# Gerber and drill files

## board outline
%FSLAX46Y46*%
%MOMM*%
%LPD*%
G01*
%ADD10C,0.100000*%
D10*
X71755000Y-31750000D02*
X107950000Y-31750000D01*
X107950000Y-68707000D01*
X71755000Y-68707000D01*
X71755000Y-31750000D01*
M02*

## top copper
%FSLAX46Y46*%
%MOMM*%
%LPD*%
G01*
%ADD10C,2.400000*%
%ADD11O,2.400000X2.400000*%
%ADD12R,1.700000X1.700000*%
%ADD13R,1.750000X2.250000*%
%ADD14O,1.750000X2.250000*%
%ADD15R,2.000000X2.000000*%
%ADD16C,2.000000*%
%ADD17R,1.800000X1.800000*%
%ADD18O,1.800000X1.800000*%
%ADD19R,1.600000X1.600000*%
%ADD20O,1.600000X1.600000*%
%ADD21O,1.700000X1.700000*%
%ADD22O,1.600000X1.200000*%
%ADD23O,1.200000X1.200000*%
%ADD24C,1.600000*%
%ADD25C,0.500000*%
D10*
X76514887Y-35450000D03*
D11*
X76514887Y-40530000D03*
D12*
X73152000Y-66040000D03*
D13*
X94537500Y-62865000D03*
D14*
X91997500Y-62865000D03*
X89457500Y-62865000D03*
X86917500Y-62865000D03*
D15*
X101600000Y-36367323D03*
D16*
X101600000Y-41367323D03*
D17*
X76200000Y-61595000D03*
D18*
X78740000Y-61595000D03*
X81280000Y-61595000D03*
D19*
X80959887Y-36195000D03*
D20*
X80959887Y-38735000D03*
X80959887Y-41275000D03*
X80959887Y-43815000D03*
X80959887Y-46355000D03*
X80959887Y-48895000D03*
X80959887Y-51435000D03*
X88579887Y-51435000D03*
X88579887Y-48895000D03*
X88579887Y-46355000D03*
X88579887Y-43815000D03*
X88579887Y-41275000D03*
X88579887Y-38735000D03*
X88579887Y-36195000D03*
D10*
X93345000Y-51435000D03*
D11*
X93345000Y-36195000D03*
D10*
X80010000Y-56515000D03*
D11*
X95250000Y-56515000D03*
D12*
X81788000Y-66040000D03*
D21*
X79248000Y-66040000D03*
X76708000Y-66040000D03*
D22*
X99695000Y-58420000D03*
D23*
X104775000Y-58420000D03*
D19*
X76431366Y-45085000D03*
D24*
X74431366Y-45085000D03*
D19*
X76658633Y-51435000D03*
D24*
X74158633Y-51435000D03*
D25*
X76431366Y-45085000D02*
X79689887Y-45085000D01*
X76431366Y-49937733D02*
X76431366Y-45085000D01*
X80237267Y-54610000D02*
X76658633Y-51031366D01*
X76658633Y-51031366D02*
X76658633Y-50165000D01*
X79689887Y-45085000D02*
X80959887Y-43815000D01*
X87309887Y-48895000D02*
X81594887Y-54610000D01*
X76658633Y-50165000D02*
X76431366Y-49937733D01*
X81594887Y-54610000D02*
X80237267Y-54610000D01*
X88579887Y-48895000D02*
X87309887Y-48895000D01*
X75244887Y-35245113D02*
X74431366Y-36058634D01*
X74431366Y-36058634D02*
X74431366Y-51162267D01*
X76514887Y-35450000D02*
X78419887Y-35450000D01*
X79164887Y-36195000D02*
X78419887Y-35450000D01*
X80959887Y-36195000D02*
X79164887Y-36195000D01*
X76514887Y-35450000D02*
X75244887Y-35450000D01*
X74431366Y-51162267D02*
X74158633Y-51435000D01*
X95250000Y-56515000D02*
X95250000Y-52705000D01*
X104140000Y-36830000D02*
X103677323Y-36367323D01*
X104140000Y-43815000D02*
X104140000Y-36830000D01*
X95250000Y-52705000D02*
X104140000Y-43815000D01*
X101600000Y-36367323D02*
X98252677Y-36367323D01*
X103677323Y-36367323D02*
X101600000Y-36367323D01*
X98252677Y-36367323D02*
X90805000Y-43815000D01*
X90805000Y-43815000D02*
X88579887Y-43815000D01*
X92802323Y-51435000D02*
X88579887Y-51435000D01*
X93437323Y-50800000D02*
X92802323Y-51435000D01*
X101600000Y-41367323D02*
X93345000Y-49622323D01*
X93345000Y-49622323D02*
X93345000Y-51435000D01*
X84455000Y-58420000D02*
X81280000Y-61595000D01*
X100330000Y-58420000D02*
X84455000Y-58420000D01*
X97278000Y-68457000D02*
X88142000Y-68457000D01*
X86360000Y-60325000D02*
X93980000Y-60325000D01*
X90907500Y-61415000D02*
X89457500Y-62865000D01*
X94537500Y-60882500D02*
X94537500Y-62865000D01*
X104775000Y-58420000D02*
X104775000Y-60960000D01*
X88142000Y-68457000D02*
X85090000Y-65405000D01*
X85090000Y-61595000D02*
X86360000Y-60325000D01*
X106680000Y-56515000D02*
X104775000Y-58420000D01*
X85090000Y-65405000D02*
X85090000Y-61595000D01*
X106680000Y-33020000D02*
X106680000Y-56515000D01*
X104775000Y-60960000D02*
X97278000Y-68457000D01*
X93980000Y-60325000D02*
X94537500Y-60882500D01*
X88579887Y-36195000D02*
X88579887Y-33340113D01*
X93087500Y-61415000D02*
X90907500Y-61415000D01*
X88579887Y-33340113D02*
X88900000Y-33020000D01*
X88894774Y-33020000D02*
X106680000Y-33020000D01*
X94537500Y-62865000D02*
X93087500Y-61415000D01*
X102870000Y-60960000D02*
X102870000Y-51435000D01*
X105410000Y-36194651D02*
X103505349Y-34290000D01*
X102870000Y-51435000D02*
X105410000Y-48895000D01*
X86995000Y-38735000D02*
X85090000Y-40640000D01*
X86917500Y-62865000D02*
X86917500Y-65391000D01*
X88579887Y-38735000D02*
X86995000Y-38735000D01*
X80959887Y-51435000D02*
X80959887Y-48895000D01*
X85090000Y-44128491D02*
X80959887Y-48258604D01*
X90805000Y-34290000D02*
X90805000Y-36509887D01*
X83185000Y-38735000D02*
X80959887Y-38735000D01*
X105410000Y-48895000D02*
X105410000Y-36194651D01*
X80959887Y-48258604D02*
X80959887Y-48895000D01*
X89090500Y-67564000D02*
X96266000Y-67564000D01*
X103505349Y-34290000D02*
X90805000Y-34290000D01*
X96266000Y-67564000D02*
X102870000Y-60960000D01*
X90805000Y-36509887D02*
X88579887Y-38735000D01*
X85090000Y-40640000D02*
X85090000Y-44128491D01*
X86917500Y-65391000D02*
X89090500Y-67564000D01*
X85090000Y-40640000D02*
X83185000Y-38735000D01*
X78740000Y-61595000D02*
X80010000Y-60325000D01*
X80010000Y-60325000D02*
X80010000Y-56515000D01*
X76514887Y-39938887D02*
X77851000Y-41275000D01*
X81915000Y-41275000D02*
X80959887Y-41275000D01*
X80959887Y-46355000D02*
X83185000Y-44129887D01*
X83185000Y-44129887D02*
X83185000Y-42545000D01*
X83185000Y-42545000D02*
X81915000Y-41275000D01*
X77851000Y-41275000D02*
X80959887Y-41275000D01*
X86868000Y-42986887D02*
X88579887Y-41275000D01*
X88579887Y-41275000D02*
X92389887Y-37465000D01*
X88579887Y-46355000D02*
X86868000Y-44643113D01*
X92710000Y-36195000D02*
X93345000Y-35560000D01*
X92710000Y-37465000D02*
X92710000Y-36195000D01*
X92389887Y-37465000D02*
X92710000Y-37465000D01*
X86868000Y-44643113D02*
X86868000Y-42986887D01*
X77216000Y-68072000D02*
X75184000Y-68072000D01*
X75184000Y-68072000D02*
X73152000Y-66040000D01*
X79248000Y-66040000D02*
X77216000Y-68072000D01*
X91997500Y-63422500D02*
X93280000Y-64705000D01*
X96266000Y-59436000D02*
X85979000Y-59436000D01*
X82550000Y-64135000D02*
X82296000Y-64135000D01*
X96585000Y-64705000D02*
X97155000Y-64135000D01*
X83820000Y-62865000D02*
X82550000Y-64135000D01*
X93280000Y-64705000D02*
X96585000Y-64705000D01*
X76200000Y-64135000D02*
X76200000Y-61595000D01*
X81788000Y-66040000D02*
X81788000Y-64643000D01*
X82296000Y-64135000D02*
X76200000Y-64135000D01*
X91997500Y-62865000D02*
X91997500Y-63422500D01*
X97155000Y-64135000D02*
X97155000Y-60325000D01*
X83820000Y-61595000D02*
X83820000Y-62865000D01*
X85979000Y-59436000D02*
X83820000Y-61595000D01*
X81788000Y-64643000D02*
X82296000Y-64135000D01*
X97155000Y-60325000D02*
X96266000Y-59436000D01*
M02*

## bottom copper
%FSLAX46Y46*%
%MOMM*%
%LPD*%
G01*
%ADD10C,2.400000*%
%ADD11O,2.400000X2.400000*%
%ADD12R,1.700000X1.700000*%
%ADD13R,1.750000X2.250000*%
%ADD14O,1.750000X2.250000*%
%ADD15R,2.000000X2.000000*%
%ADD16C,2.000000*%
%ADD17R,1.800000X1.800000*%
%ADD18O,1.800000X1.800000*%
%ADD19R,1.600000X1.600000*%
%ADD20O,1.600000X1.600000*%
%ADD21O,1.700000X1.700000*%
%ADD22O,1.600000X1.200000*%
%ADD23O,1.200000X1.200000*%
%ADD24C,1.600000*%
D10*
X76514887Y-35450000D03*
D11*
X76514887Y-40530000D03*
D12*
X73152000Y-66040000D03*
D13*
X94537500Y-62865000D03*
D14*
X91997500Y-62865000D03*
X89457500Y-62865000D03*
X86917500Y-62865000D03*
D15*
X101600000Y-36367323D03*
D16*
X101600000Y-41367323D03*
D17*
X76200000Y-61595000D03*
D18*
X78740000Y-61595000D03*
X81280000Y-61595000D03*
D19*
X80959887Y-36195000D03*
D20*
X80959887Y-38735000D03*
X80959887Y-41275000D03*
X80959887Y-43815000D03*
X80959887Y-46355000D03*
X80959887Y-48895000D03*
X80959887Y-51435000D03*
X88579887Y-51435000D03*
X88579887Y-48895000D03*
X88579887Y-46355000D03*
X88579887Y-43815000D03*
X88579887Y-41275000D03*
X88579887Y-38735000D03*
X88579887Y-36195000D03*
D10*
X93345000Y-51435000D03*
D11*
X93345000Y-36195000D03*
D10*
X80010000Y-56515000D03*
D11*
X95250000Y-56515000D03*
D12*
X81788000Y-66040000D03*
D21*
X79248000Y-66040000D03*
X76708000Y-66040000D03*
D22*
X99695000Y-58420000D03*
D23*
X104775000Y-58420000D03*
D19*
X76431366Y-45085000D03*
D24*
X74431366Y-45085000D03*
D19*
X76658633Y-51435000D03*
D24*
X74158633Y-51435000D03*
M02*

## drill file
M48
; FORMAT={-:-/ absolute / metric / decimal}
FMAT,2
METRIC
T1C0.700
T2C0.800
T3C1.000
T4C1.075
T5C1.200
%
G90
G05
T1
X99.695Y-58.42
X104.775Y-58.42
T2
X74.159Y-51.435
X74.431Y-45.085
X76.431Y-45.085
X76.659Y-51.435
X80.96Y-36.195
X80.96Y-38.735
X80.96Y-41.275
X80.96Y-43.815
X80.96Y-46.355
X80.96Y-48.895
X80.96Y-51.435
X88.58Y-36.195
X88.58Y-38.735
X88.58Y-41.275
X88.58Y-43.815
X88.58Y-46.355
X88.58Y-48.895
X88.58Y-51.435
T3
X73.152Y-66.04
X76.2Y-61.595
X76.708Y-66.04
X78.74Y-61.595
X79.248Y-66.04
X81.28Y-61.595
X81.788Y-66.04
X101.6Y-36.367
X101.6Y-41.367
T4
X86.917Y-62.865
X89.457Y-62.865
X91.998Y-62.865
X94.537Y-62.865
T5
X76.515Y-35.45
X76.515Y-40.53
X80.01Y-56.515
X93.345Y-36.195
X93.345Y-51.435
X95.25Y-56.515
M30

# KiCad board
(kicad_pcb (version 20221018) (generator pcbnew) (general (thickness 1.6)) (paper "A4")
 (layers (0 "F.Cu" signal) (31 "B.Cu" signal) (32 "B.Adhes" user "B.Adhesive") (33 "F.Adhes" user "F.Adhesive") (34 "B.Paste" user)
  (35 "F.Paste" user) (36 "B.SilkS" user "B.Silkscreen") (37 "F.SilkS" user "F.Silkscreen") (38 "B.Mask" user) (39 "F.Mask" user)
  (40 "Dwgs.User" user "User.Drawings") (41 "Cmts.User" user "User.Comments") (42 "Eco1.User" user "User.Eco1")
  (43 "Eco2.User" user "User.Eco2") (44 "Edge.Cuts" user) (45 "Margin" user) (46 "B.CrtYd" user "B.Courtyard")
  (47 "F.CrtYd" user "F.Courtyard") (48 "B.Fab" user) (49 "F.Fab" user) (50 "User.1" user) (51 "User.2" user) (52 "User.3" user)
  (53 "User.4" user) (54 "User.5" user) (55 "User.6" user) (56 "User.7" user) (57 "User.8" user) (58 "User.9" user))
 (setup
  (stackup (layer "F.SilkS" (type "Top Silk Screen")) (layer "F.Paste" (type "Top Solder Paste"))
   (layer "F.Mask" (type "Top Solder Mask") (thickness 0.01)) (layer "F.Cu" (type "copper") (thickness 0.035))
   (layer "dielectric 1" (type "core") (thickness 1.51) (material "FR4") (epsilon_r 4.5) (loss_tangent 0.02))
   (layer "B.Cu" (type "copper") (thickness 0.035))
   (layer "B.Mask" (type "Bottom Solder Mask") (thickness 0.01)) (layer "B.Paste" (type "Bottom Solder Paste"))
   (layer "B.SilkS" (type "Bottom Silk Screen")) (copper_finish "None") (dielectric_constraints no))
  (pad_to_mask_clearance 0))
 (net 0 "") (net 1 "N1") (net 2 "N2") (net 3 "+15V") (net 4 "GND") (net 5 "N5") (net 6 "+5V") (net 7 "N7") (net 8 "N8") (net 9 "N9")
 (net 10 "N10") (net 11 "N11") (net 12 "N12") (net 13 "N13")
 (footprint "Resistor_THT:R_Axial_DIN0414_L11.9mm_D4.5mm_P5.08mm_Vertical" (layer "F.Cu") (at 76.514887 35.45 -90)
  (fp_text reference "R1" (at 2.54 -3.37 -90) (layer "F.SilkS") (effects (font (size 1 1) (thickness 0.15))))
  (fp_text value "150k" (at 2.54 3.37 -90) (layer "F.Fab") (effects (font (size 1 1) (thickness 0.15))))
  (pad "1" thru_hole circle (at 0 0 270) (size 2.4 2.4) (drill 1.2) (layers "*.Cu" "*.Mask") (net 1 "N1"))
  (pad "2" thru_hole oval (at 5.08 0 270) (size 2.4 2.4) (drill 1.2) (layers "*.Cu" "*.Mask") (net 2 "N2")))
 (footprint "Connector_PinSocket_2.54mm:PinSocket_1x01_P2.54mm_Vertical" (layer "F.Cu") (at 73.152 66.04)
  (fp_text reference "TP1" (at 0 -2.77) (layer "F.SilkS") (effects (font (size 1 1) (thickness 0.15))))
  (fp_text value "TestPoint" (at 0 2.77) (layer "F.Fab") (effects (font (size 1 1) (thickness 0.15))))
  (pad "1" thru_hole rect (at 0 0) (size 1.7 1.7) (drill 1) (layers "*.Cu" "*.Mask") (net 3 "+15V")))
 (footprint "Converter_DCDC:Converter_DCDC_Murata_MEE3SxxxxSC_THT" (layer "F.Cu") (at 94.5375 62.865 -90)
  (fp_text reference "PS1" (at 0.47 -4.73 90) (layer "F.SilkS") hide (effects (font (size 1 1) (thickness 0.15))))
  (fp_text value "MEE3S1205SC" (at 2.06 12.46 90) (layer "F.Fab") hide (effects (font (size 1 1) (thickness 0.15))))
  (pad "1" thru_hole rect (at 0 0 180) (size 1.75 2.25) (drill 1.075) (layers "*.Cu" "*.Mask") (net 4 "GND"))
  (pad "2" thru_hole oval (at 0 2.54 180) (size 1.75 2.25) (drill 1.075) (layers "*.Cu" "*.Mask") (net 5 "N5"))
  (pad "3" thru_hole oval (at 0 5.08 180) (size 1.75 2.25) (drill 1.075) (layers "*.Cu" "*.Mask") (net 4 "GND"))
  (pad "4" thru_hole oval (at 0 7.62 180) (size 1.75 2.25) (drill 1.075) (layers "*.Cu" "*.Mask") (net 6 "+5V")))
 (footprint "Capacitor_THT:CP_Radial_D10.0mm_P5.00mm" (layer "F.Cu") (at 101.6 36.367323 -90)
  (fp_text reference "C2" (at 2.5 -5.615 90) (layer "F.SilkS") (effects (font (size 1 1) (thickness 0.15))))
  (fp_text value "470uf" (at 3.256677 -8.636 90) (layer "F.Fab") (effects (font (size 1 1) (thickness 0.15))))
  (pad "1" thru_hole rect (at 0 0 270) (size 2 2) (drill 1) (layers "*.Cu" "*.Mask") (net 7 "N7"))
  (pad "2" thru_hole circle (at 5 0 270) (size 2 2) (drill 1) (layers "*.Cu" "*.Mask") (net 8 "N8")))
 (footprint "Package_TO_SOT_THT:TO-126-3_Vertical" (layer "F.Cu") (at 76.2 61.595)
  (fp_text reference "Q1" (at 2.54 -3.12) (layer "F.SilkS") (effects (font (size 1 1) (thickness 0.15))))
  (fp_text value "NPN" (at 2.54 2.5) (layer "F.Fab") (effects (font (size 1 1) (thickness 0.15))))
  (pad "1" thru_hole rect (at 0 0) (size 1.8 1.8) (drill 1) (layers "*.Cu" "*.Mask") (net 5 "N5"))
  (pad "2" thru_hole oval (at 2.54 0) (size 1.8 1.8) (drill 1) (layers "*.Cu" "*.Mask") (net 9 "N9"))
  (pad "3" thru_hole oval (at 5.08 0) (size 1.8 1.8) (drill 1) (layers "*.Cu" "*.Mask") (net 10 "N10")))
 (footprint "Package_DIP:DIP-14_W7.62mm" (layer "F.Cu") (at 80.959887 36.195)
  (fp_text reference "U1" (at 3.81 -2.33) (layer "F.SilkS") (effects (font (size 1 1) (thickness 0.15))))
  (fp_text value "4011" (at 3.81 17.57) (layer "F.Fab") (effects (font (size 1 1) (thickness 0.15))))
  (pad "1" thru_hole rect (at 0 0) (size 1.6 1.6) (drill 0.8) (layers "*.Cu" "*.Mask") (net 1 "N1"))
  (pad "2" thru_hole oval (at 0 2.54) (size 1.6 1.6) (drill 0.8) (layers "*.Cu" "*.Mask") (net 6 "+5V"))
  (pad "3" thru_hole oval (at 0 5.08) (size 1.6 1.6) (drill 0.8) (layers "*.Cu" "*.Mask") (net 2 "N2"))
  (pad "4" thru_hole oval (at 0 7.62) (size 1.6 1.6) (drill 0.8) (layers "*.Cu" "*.Mask") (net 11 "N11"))
  (pad "5" thru_hole oval (at 0 10.16) (size 1.6 1.6) (drill 0.8) (layers "*.Cu" "*.Mask") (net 2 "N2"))
  (pad "6" thru_hole oval (at 0 12.7) (size 1.6 1.6) (drill 0.8) (layers "*.Cu" "*.Mask") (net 6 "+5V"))
  (pad "7" thru_hole oval (at 0 15.24) (size 1.6 1.6) (drill 0.8) (layers "*.Cu" "*.Mask") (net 6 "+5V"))
  (pad "8" thru_hole oval (at 7.62 15.24) (size 1.6 1.6) (drill 0.8) (layers "*.Cu" "*.Mask") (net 8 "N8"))
  (pad "9" thru_hole oval (at 7.62 12.7) (size 1.6 1.6) (drill 0.8) (layers "*.Cu" "*.Mask") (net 11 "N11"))
  (pad "10" thru_hole oval (at 7.62 10.16) (size 1.6 1.6) (drill 0.8) (layers "*.Cu" "*.Mask") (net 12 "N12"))
  (pad "11" thru_hole oval (at 7.62 7.62) (size 1.6 1.6) (drill 0.8) (layers "*.Cu" "*.Mask") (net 7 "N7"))
  (pad "12" thru_hole oval (at 7.62 5.08) (size 1.6 1.6) (drill 0.8) (layers "*.Cu" "*.Mask") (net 12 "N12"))
  (pad "13" thru_hole oval (at 7.62 2.54) (size 1.6 1.6) (drill 0.8) (layers "*.Cu" "*.Mask") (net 6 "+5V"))
  (pad "14" thru_hole oval (at 7.62 0) (size 1.6 1.6) (drill 0.8) (layers "*.Cu" "*.Mask") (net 4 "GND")))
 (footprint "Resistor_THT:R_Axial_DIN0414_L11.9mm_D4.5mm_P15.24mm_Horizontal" (layer "F.Cu") (at 93.345 51.435 90)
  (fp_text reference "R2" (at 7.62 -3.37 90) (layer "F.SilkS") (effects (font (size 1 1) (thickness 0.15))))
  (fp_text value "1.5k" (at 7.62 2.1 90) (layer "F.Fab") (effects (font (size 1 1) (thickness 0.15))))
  (pad "1" thru_hole circle (at 0 0 90) (size 2.4 2.4) (drill 1.2) (layers "*.Cu" "*.Mask") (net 8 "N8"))
  (pad "2" thru_hole oval (at 15.24 0 90) (size 2.4 2.4) (drill 1.2) (layers "*.Cu" "*.Mask") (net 12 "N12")))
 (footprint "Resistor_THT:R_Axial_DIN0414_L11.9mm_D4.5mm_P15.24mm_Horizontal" (layer "F.Cu") (at 80.01 56.515)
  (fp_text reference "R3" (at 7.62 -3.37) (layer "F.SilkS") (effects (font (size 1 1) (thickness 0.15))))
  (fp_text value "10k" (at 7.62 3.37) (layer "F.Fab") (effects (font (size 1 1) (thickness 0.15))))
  (pad "1" thru_hole circle (at 0 0) (size 2.4 2.4) (drill 1.2) (layers "*.Cu" "*.Mask") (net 9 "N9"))
  (pad "2" thru_hole oval (at 15.24 0) (size 2.4 2.4) (drill 1.2) (layers "*.Cu" "*.Mask") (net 7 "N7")))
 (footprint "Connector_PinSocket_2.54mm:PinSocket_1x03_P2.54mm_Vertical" (layer "F.Cu") (at 81.788 66.04 -90)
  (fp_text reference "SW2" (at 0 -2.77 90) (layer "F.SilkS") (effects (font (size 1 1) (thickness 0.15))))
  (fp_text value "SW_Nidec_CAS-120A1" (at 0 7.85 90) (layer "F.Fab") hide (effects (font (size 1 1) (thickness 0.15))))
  (pad "1" thru_hole rect (at 0 0 270) (size 1.7 1.7) (drill 1) (layers "*.Cu" "*.Mask") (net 5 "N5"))
  (pad "2" thru_hole oval (at 0 2.54 270) (size 1.7 1.7) (drill 1) (layers "*.Cu" "*.Mask") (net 3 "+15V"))
  (pad "3" thru_hole oval (at 0 5.08 270) (size 1.7 1.7) (drill 1) (layers "*.Cu" "*.Mask") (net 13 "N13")))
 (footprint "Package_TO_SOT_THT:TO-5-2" (layer "F.Cu") (at 99.695 58.42)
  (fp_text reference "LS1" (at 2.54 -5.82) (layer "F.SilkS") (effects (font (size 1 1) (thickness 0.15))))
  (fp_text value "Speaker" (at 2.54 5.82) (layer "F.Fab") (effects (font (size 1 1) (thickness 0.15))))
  (pad "1" thru_hole oval (at 0 0) (size 1.6 1.2) (drill 0.7) (layers "*.Cu" "*.Mask") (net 10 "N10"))
  (pad "2" thru_hole oval (at 5.08 0) (size 1.2 1.2) (drill 0.7) (layers "*.Cu" "*.Mask") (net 4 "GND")))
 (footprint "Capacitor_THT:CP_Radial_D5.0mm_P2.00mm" (layer "F.Cu") (at 76.431366 45.085 180)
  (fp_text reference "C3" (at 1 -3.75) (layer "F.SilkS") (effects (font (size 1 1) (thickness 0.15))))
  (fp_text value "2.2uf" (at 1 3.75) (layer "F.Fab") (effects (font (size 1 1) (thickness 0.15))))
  (pad "1" thru_hole rect (at 0 0 180) (size 1.6 1.6) (drill 0.8) (layers "*.Cu" "*.Mask") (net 11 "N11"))
  (pad "2" thru_hole circle (at 2 0 180) (size 1.6 1.6) (drill 0.8) (layers "*.Cu" "*.Mask") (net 1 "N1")))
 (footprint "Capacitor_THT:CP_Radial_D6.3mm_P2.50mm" (layer "F.Cu") (at 76.658633 51.435 180)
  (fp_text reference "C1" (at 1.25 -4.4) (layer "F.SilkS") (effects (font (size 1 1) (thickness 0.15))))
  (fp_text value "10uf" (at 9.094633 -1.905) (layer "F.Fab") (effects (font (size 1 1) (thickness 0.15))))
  (pad "1" thru_hole rect (at 0 0 180) (size 1.6 1.6) (drill 0.8) (layers "*.Cu" "*.Mask") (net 11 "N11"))
  (pad "2" thru_hole circle (at 2.5 0 180) (size 1.6 1.6) (drill 0.8) (layers "*.Cu" "*.Mask") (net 1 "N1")))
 (gr_rect (start 71.755 31.75) (end 107.95 68.707) (stroke (width 0.1) (type default)) (fill none) (layer "Edge.Cuts"))
 (segment (start 76.431366 45.085) (end 79.689887 45.085) (width 0.5) (layer "F.Cu") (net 11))
 (segment (start 76.431366 49.937733) (end 76.431366 45.085) (width 0.5) (layer "F.Cu") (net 11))
 (segment (start 80.237267 54.61) (end 76.658633 51.031366) (width 0.5) (layer "F.Cu") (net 11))
 (segment (start 76.658633 51.031366) (end 76.658633 50.165) (width 0.5) (layer "F.Cu") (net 11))
 (segment (start 79.689887 45.085) (end 80.959887 43.815) (width 0.5) (layer "F.Cu") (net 11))
 (segment (start 87.309887 48.895) (end 81.594887 54.61) (width 0.5) (layer "F.Cu") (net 11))
 (segment (start 76.658633 50.165) (end 76.431366 49.937733) (width 0.5) (layer "F.Cu") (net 11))
 (segment (start 81.594887 54.61) (end 80.237267 54.61) (width 0.5) (layer "F.Cu") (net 11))
 (segment (start 88.579887 48.895) (end 87.309887 48.895) (width 0.5) (layer "F.Cu") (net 11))
 (segment (start 75.244887 35.245113) (end 74.431366 36.058634) (width 0.5) (layer "F.Cu") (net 1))
 (segment (start 74.431366 36.058634) (end 74.431366 51.162267) (width 0.5) (layer "F.Cu") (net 1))
 (segment (start 76.514887 35.45) (end 78.419887 35.45) (width 0.5) (layer "F.Cu") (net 1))
 (segment (start 79.164887 36.195) (end 78.419887 35.45) (width 0.5) (layer "F.Cu") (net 1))
 (segment (start 80.959887 36.195) (end 79.164887 36.195) (width 0.5) (layer "F.Cu") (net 1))
 (segment (start 76.514887 35.45) (end 75.244887 35.45) (width 0.5) (layer "F.Cu") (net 1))
 (segment (start 74.431366 51.162267) (end 74.158633 51.435) (width 0.5) (layer "F.Cu") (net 1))
 (segment (start 95.25 56.515) (end 95.25 52.705) (width 0.5) (layer "F.Cu") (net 7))
 (segment (start 104.14 36.83) (end 103.677323 36.367323) (width 0.5) (layer "F.Cu") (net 7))
 (segment (start 104.14 43.815) (end 104.14 36.83) (width 0.5) (layer "F.Cu") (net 7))
 (segment (start 95.25 52.705) (end 104.14 43.815) (width 0.5) (layer "F.Cu") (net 7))
 (segment (start 101.6 36.367323) (end 98.252677 36.367323) (width 0.5) (layer "F.Cu") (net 7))
 (segment (start 103.677323 36.367323) (end 101.6 36.367323) (width 0.5) (layer "F.Cu") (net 7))
 (segment (start 98.252677 36.367323) (end 90.805 43.815) (width 0.5) (layer "F.Cu") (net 7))
 (segment (start 90.805 43.815) (end 88.579887 43.815) (width 0.5) (layer "F.Cu") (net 7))
 (segment (start 92.802323 51.435) (end 88.579887 51.435) (width 0.5) (layer "F.Cu") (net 8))
 (segment (start 93.437323 50.8) (end 92.802323 51.435) (width 0.5) (layer "F.Cu") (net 8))
 (segment (start 101.6 41.367323) (end 93.345 49.622323) (width 0.5) (layer "F.Cu") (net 8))
 (segment (start 93.345 49.622323) (end 93.345 51.435) (width 0.5) (layer "F.Cu") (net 8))
 (segment (start 84.455 58.42) (end 81.28 61.595) (width 0.5) (layer "F.Cu") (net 10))
 (segment (start 100.33 58.42) (end 84.455 58.42) (width 0.5) (layer "F.Cu") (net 10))
 (segment (start 97.278 68.457) (end 88.142 68.457) (width 0.5) (layer "F.Cu") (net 4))
 (segment (start 86.36 60.325) (end 93.98 60.325) (width 0.5) (layer "F.Cu") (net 4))
 (segment (start 90.9075 61.415) (end 89.4575 62.865) (width 0.5) (layer "F.Cu") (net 4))
 (segment (start 94.5375 60.8825) (end 94.5375 62.865) (width 0.5) (layer "F.Cu") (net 4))
 (segment (start 104.775 58.42) (end 104.775 60.96) (width 0.5) (layer "F.Cu") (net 4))
 (segment (start 88.142 68.457) (end 85.09 65.405) (width 0.5) (layer "F.Cu") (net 4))
 (segment (start 85.09 61.595) (end 86.36 60.325) (width 0.5) (layer "F.Cu") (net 4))
 (segment (start 106.68 56.515) (end 104.775 58.42) (width 0.5) (layer "F.Cu") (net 4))
 (segment (start 85.09 65.405) (end 85.09 61.595) (width 0.5) (layer "F.Cu") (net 4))
 (segment (start 106.68 33.02) (end 106.68 56.515) (width 0.5) (layer "F.Cu") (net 4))
 (segment (start 104.775 60.96) (end 97.278 68.457) (width 0.5) (layer "F.Cu") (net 4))
 (segment (start 93.98 60.325) (end 94.5375 60.8825) (width 0.5) (layer "F.Cu") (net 4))
 (segment (start 88.579887 36.195) (end 88.579887 33.340113) (width 0.5) (layer "F.Cu") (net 4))
 (segment (start 93.0875 61.415) (end 90.9075 61.415) (width 0.5) (layer "F.Cu") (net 4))
 (segment (start 88.579887 33.340113) (end 88.9 33.02) (width 0.5) (layer "F.Cu") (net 4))
 (segment (start 88.894774 33.02) (end 106.68 33.02) (width 0.5) (layer "F.Cu") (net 4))
 (segment (start 94.5375 62.865) (end 93.0875 61.415) (width 0.5) (layer "F.Cu") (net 4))
 (segment (start 102.87 60.96) (end 102.87 51.435) (width 0.5) (layer "F.Cu") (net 6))
 (segment (start 105.41 36.194651) (end 103.505349 34.29) (width 0.5) (layer "F.Cu") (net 6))
 (segment (start 102.87 51.435) (end 105.41 48.895) (width 0.5) (layer "F.Cu") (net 6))
 (segment (start 86.995 38.735) (end 85.09 40.64) (width 0.5) (layer "F.Cu") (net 6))
 (segment (start 86.9175 62.865) (end 86.9175 65.391) (width 0.5) (layer "F.Cu") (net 6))
 (segment (start 88.579887 38.735) (end 86.995 38.735) (width 0.5) (layer "F.Cu") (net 6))
 (segment (start 80.959887 51.435) (end 80.959887 48.895) (width 0.5) (layer "F.Cu") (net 6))
 (segment (start 85.09 44.128491) (end 80.959887 48.258604) (width 0.5) (layer "F.Cu") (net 6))
 (segment (start 90.805 34.29) (end 90.805 36.509887) (width 0.5) (layer "F.Cu") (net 6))
 (segment (start 83.185 38.735) (end 80.959887 38.735) (width 0.5) (layer "F.Cu") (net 6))
 (segment (start 105.41 48.895) (end 105.41 36.194651) (width 0.5) (layer "F.Cu") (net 6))
 (segment (start 80.959887 48.258604) (end 80.959887 48.895) (width 0.5) (layer "F.Cu") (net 6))
 (segment (start 89.0905 67.564) (end 96.266 67.564) (width 0.5) (layer "F.Cu") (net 6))
 (segment (start 103.505349 34.29) (end 90.805 34.29) (width 0.5) (layer "F.Cu") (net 6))
 (segment (start 96.266 67.564) (end 102.87 60.96) (width 0.5) (layer "F.Cu") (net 6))
 (segment (start 90.805 36.509887) (end 88.579887 38.735) (width 0.5) (layer "F.Cu") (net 6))
 (segment (start 85.09 40.64) (end 85.09 44.128491) (width 0.5) (layer "F.Cu") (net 6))
 (segment (start 86.9175 65.391) (end 89.0905 67.564) (width 0.5) (layer "F.Cu") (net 6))
 (segment (start 85.09 40.64) (end 83.185 38.735) (width 0.5) (layer "F.Cu") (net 6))
 (segment (start 78.74 61.595) (end 80.01 60.325) (width 0.5) (layer "F.Cu") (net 9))
 (segment (start 80.01 60.325) (end 80.01 56.515) (width 0.5) (layer "F.Cu") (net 9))
 (segment (start 76.514887 39.938887) (end 77.851 41.275) (width 0.5) (layer "F.Cu") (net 2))
 (segment (start 81.915 41.275) (end 80.959887 41.275) (width 0.5) (layer "F.Cu") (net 2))
 (segment (start 80.959887 46.355) (end 83.185 44.129887) (width 0.5) (layer "F.Cu") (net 2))
 (segment (start 83.185 44.129887) (end 83.185 42.545) (width 0.5) (layer "F.Cu") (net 2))
 (segment (start 83.185 42.545) (end 81.915 41.275) (width 0.5) (layer "F.Cu") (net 2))
 (segment (start 77.851 41.275) (end 80.959887 41.275) (width 0.5) (layer "F.Cu") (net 2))
 (segment (start 86.868 42.986887) (end 88.579887 41.275) (width 0.5) (layer "F.Cu") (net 12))
 (segment (start 88.579887 41.275) (end 92.389887 37.465) (width 0.5) (layer "F.Cu") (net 12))
 (segment (start 88.579887 46.355) (end 86.868 44.643113) (width 0.5) (layer "F.Cu") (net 12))
 (segment (start 92.71 36.195) (end 93.345 35.56) (width 0.5) (layer "F.Cu") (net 12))
 (segment (start 92.71 37.465) (end 92.71 36.195) (width 0.5) (layer "F.Cu") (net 12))
 (segment (start 92.389887 37.465) (end 92.71 37.465) (width 0.5) (layer "F.Cu") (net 12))
 (segment (start 86.868 44.643113) (end 86.868 42.986887) (width 0.5) (layer "F.Cu") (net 12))
 (segment (start 77.216 68.072) (end 75.184 68.072) (width 0.5) (layer "F.Cu") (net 3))
 (segment (start 75.184 68.072) (end 73.152 66.04) (width 0.5) (layer "F.Cu") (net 3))
 (segment (start 79.248 66.04) (end 77.216 68.072) (width 0.5) (layer "F.Cu") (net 3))
 (segment (start 91.9975 63.4225) (end 93.28 64.705) (width 0.5) (layer "F.Cu") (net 5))
 (segment (start 96.266 59.436) (end 85.979 59.436) (width 0.5) (layer "F.Cu") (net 5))
 (segment (start 82.55 64.135) (end 82.296 64.135) (width 0.5) (layer "F.Cu") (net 5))
 (segment (start 96.585 64.705) (end 97.155 64.135) (width 0.5) (layer "F.Cu") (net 5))
 (segment (start 83.82 62.865) (end 82.55 64.135) (width 0.5) (layer "F.Cu") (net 5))
 (segment (start 93.28 64.705) (end 96.585 64.705) (width 0.5) (layer "F.Cu") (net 5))
 (segment (start 76.2 64.135) (end 76.2 61.595) (width 0.5) (layer "F.Cu") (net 5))
 (segment (start 81.788 66.04) (end 81.788 64.643) (width 0.5) (layer "F.Cu") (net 5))
 (segment (start 82.296 64.135) (end 76.2 64.135) (width 0.5) (layer "F.Cu") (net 5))
 (segment (start 91.9975 62.865) (end 91.9975 63.4225) (width 0.5) (layer "F.Cu") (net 5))
 (segment (start 97.155 64.135) (end 97.155 60.325) (width 0.5) (layer "F.Cu") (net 5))
 (segment (start 83.82 61.595) (end 83.82 62.865) (width 0.5) (layer "F.Cu") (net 5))
 (segment (start 85.979 59.436) (end 83.82 61.595) (width 0.5) (layer "F.Cu") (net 5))
 (segment (start 81.788 64.643) (end 82.296 64.135) (width 0.5) (layer "F.Cu") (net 5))
 (segment (start 97.155 60.325) (end 96.266 59.436) (width 0.5) (layer "F.Cu") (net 5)))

